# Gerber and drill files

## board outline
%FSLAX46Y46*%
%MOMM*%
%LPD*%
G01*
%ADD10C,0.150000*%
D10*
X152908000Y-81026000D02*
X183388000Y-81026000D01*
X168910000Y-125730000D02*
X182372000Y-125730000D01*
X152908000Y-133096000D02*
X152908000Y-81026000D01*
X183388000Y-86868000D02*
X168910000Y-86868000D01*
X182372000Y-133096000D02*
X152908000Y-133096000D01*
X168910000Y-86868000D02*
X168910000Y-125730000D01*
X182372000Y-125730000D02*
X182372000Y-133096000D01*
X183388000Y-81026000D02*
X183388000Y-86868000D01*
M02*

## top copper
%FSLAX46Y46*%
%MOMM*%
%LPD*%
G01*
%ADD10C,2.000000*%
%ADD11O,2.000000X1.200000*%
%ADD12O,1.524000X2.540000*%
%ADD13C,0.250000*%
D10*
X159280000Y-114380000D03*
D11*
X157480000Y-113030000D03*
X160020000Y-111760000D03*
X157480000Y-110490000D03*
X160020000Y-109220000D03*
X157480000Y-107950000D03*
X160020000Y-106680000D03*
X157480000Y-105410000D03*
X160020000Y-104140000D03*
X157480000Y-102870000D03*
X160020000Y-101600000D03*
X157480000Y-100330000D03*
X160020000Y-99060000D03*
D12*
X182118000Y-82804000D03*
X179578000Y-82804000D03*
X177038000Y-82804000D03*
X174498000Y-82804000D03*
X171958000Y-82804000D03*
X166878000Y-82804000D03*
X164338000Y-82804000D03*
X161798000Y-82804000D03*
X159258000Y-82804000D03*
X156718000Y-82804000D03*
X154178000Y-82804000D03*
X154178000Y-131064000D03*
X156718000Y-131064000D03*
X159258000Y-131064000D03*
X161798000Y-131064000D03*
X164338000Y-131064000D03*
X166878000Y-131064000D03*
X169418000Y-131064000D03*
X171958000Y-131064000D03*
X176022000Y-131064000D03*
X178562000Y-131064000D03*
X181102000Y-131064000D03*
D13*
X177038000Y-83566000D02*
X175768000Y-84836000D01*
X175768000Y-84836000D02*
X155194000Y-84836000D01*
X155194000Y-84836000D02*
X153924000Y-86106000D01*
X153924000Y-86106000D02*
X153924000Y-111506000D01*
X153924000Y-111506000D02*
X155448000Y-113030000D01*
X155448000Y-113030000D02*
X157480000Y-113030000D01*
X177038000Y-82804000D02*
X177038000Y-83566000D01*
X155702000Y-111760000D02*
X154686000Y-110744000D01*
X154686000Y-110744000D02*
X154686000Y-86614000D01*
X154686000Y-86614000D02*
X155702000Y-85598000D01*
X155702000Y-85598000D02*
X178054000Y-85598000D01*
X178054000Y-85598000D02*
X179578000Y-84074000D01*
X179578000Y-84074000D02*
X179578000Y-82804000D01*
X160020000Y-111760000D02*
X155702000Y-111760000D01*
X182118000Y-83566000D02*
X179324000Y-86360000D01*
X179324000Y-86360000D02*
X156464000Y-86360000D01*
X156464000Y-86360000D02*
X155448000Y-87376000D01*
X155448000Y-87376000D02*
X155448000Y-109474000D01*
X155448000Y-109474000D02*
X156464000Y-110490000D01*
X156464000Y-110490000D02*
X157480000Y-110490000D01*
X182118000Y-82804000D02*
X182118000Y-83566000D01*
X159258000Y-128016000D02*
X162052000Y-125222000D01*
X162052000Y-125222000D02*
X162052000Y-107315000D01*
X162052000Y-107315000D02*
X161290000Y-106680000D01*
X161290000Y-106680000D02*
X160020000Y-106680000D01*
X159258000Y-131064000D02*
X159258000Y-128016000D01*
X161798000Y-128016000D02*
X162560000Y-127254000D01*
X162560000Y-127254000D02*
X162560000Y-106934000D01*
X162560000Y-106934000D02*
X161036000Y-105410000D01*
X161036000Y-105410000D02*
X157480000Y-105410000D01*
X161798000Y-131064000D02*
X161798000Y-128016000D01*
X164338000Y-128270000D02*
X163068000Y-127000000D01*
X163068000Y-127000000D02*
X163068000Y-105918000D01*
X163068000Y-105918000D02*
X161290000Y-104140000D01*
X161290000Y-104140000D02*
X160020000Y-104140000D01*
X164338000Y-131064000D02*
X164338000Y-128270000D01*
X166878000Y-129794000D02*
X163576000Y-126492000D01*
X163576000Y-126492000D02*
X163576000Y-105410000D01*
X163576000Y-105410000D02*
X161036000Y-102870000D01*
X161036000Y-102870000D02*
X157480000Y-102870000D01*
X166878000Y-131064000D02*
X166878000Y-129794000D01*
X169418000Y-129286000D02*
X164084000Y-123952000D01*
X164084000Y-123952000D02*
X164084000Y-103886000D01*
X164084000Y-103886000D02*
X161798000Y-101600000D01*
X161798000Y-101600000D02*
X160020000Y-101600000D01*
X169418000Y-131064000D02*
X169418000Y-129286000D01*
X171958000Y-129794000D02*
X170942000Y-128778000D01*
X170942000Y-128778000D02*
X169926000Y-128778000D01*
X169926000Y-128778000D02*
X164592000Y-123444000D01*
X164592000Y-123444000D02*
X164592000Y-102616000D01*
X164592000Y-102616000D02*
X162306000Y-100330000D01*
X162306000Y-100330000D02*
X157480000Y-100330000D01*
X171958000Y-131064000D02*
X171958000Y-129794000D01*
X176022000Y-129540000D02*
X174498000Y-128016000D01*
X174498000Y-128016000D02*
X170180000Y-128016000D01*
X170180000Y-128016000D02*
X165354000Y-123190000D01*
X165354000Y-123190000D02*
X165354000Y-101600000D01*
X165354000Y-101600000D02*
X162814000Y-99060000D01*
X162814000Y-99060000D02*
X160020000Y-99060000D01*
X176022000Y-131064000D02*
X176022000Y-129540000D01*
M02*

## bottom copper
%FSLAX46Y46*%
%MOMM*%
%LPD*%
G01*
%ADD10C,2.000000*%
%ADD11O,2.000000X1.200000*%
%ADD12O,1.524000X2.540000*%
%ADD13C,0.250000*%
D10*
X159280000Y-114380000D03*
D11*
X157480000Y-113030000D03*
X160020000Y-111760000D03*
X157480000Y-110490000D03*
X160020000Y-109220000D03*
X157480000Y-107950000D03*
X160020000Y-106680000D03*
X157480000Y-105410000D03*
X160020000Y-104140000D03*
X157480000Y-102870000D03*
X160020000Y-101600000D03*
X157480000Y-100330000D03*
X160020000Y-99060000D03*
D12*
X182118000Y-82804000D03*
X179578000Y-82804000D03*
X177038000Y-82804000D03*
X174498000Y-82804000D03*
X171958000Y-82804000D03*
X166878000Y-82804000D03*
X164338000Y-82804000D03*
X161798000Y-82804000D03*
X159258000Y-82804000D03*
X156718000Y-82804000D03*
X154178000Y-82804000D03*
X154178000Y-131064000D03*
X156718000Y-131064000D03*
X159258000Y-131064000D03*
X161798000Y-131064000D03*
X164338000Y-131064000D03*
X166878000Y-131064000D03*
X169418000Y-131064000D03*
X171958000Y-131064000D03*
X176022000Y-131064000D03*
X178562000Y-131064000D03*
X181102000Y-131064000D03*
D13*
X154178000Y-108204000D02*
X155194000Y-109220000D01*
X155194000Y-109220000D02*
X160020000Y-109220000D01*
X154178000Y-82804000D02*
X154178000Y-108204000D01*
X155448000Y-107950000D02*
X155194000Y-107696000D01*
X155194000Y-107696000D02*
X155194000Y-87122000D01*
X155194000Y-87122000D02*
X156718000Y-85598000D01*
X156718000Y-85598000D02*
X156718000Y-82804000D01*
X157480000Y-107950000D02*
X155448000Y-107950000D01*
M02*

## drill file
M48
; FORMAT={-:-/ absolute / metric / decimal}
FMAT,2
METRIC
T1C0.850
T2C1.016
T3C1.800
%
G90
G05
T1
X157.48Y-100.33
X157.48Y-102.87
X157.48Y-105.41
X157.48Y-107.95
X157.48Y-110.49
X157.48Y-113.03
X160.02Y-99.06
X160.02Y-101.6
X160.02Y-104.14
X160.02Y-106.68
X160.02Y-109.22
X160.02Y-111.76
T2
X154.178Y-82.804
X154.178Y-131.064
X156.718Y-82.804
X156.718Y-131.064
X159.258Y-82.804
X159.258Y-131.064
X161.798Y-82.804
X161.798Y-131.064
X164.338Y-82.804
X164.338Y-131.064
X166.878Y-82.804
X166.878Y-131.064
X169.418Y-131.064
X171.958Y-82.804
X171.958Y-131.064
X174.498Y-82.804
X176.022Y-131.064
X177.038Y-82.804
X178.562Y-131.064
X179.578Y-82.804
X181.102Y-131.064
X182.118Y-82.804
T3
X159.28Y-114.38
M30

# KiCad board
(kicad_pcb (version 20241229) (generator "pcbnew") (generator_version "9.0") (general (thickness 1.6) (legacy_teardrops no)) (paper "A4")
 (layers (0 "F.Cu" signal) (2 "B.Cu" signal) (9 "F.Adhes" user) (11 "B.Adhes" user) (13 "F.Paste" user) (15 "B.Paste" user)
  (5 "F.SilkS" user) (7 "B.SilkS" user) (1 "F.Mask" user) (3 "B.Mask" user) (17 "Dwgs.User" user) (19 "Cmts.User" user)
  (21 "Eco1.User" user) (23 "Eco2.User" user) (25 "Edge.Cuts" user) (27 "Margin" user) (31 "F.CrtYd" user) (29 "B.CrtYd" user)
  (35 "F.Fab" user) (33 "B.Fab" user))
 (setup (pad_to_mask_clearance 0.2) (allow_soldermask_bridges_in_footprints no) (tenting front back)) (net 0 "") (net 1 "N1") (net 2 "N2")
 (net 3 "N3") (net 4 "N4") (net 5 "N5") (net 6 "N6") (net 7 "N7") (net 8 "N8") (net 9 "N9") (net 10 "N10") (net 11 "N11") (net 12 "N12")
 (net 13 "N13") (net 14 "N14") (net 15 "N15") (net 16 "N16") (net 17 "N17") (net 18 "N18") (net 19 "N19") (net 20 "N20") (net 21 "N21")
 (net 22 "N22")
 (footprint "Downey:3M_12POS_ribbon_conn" (layer "F.Cu") (at 158.75 106.68 90)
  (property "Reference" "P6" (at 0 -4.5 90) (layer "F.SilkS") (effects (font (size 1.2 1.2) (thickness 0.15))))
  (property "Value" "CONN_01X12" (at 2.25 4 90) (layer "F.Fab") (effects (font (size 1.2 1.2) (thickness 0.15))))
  (pad "" np_thru_hole circle (at -7.7 0.53 90) (size 2 2) (drill 1.8) (layers "*.Cu" "*.Mask"))
  (pad "1" thru_hole oval (at -6.35 -1.27 90) (size 1.2 2) (drill 0.85) (layers "*.Cu" "*.Mask") (remove_unused_layers no) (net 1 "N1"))
  (pad "2" thru_hole oval (at -5.08 1.27 90) (size 1.2 2) (drill 0.85) (layers "*.Cu" "*.Mask") (remove_unused_layers no) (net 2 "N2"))
  (pad "3" thru_hole oval (at -3.81 -1.27 90) (size 1.2 2) (drill 0.85) (layers "*.Cu" "*.Mask") (remove_unused_layers no) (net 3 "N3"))
  (pad "4" thru_hole oval (at -2.54 1.27 90) (size 1.2 2) (drill 0.85) (layers "*.Cu" "*.Mask") (remove_unused_layers no) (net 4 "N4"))
  (pad "5" thru_hole oval (at -1.27 -1.27 90) (size 1.2 2) (drill 0.85) (layers "*.Cu" "*.Mask") (remove_unused_layers no) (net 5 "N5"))
  (pad "6" thru_hole oval (at 0 1.27 90) (size 1.2 2) (drill 0.85) (layers "*.Cu" "*.Mask") (remove_unused_layers no) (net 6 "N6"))
  (pad "7" thru_hole oval (at 1.27 -1.27 90) (size 1.2 2) (drill 0.85) (layers "*.Cu" "*.Mask") (remove_unused_layers no) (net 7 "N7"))
  (pad "8" thru_hole oval (at 2.54 1.27 90) (size 1.2 2) (drill 0.85) (layers "*.Cu" "*.Mask") (remove_unused_layers no) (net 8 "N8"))
  (pad "9" thru_hole oval (at 3.81 -1.27 90) (size 1.2 2) (drill 0.85) (layers "*.Cu" "*.Mask") (remove_unused_layers no) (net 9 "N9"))
  (pad "10" thru_hole oval (at 5.08 1.27 90) (size 1.2 2) (drill 0.85) (layers "*.Cu" "*.Mask") (remove_unused_layers no) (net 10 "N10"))
  (pad "11" thru_hole oval (at 6.35 -1.27 90) (size 1.2 2) (drill 0.85) (layers "*.Cu" "*.Mask") (remove_unused_layers no) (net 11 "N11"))
  (pad "12" thru_hole oval (at 7.62 1.27 90) (size 1.2 2) (drill 0.85) (layers "*.Cu" "*.Mask") (remove_unused_layers no) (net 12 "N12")))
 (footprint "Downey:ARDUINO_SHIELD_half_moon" (layer "F.Cu") (at 148.59 104.14 -90)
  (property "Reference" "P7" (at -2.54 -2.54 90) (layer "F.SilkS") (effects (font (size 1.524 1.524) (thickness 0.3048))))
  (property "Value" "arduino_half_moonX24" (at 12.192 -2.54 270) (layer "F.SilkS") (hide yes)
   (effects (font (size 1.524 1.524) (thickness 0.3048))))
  (pad "1" thru_hole oval (at -21.336 -33.528 270) (size 2.54 1.524) (drill 1.016) (layers "*.Cu" "*.Mask" "F.SilkS")
   (remove_unused_layers no) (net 3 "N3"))
  (pad "2" thru_hole oval (at -21.336 -30.988 270) (size 2.54 1.524) (drill 1.016) (layers "*.Cu" "*.Mask" "F.SilkS")
   (remove_unused_layers no) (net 2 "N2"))
  (pad "3" thru_hole oval (at -21.336 -28.448 270) (size 2.54 1.524) (drill 1.016) (layers "*.Cu" "*.Mask" "F.SilkS")
   (remove_unused_layers no) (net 1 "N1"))
  (pad "4" thru_hole oval (at -21.336 -25.908 270) (size 2.54 1.524) (drill 1.016) (layers "*.Cu" "*.Mask" "F.SilkS")
   (remove_unused_layers no) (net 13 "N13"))
  (pad "5" thru_hole oval (at -21.336 -23.368 270) (size 2.54 1.524) (drill 1.016) (layers "*.Cu" "*.Mask" "F.SilkS")
   (remove_unused_layers no) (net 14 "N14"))
  (pad "6" thru_hole oval (at -21.336 -18.288 270) (size 2.54 1.524) (drill 1.016) (layers "*.Cu" "*.Mask" "F.SilkS")
   (remove_unused_layers no) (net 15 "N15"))
  (pad "7" thru_hole oval (at -21.336 -15.748 270) (size 2.54 1.524) (drill 1.016) (layers "*.Cu" "*.Mask" "F.SilkS")
   (remove_unused_layers no) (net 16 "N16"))
  (pad "8" thru_hole oval (at -21.336 -13.208 270) (size 2.54 1.524) (drill 1.016) (layers "*.Cu" "*.Mask" "F.SilkS")
   (remove_unused_layers no) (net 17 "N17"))
  (pad "9" thru_hole oval (at -21.336 -10.668 270) (size 2.54 1.524) (drill 1.016) (layers "*.Cu" "*.Mask" "F.SilkS")
   (remove_unused_layers no) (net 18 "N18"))
  (pad "10" thru_hole oval (at -21.336 -8.128 270) (size 2.54 1.524) (drill 1.016) (layers "*.Cu" "*.Mask" "F.SilkS")
   (remove_unused_layers no) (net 5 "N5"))
  (pad "11" thru_hole oval (at -21.336 -5.588 270) (size 2.54 1.524) (drill 1.016) (layers "*.Cu" "*.Mask" "F.SilkS")
   (remove_unused_layers no) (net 4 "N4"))
  (pad "12" thru_hole oval (at 26.924 -5.588 270) (size 2.54 1.524) (drill 1.016) (layers "*.Cu" "*.Mask" "F.SilkS")
   (remove_unused_layers no) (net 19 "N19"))
  (pad "13" thru_hole oval (at 26.924 -8.128 270) (size 2.54 1.524) (drill 1.016) (layers "*.Cu" "*.Mask" "F.SilkS")
   (remove_unused_layers no) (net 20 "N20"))
  (pad "14" thru_hole oval (at 26.924 -10.668 270) (size 2.54 1.524) (drill 1.016) (layers "*.Cu" "*.Mask" "F.SilkS")
   (remove_unused_layers no) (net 6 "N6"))
  (pad "15" thru_hole oval (at 26.924 -13.208 270) (size 2.54 1.524) (drill 1.016) (layers "*.Cu" "*.Mask" "F.SilkS")
   (remove_unused_layers no) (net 7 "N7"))
  (pad "16" thru_hole oval (at 26.924 -15.748 270) (size 2.54 1.524) (drill 1.016) (layers "*.Cu" "*.Mask" "F.SilkS")
   (remove_unused_layers no) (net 8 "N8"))
  (pad "17" thru_hole oval (at 26.924 -18.288 270) (size 2.54 1.524) (drill 1.016) (layers "*.Cu" "*.Mask" "F.SilkS")
   (remove_unused_layers no) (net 9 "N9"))
  (pad "18" thru_hole oval (at 26.924 -20.828 270) (size 2.54 1.524) (drill 1.016) (layers "*.Cu" "*.Mask" "F.SilkS")
   (remove_unused_layers no) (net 10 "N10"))
  (pad "19" thru_hole oval (at 26.924 -23.368 270) (size 2.54 1.524) (drill 1.016) (layers "*.Cu" "*.Mask" "F.SilkS")
   (remove_unused_layers no) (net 11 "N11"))
  (pad "20" thru_hole oval (at 26.924 -27.432 270) (size 2.54 1.524) (drill 1.016) (layers "*.Cu" "*.Mask" "F.SilkS")
   (remove_unused_layers no) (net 12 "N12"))
  (pad "21" thru_hole oval (at 26.924 -29.972 270) (size 2.54 1.524) (drill 1.016) (layers "*.Cu" "*.Mask" "F.SilkS")
   (remove_unused_layers no) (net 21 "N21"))
  (pad "22" thru_hole oval (at 26.924 -32.512 270) (size 2.54 1.524) (drill 1.016) (layers "*.Cu" "*.Mask" "F.SilkS")
   (remove_unused_layers no) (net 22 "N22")))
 (gr_line (start 152.908 81.026) (end 183.388 81.026) (stroke (width 0.15) (type solid)) (layer "Edge.Cuts"))
 (gr_line (start 168.91 125.73) (end 182.372 125.73) (stroke (width 0.15) (type solid)) (layer "Edge.Cuts"))
 (gr_line (start 152.908 133.096) (end 152.908 81.026) (stroke (width 0.15) (type solid)) (layer "Edge.Cuts"))
 (gr_line (start 183.388 86.868) (end 168.91 86.868) (stroke (width 0.15) (type solid)) (layer "Edge.Cuts"))
 (gr_line (start 182.372 133.096) (end 152.908 133.096) (stroke (width 0.15) (type solid)) (layer "Edge.Cuts"))
 (gr_line (start 168.91 86.868) (end 168.91 125.73) (stroke (width 0.15) (type solid)) (layer "Edge.Cuts"))
 (gr_line (start 182.372 125.73) (end 182.372 133.096) (stroke (width 0.15) (type solid)) (layer "Edge.Cuts"))
 (gr_line (start 183.388 81.026) (end 183.388 86.868) (stroke (width 0.15) (type solid)) (layer "Edge.Cuts"))
 (segment (start 177.038 83.566) (end 175.768 84.836) (width 0.25) (layer "F.Cu") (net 1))
 (segment (start 175.768 84.836) (end 155.194 84.836) (width 0.25) (layer "F.Cu") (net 1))
 (segment (start 155.194 84.836) (end 153.924 86.106) (width 0.25) (layer "F.Cu") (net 1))
 (segment (start 153.924 86.106) (end 153.924 111.506) (width 0.25) (layer "F.Cu") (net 1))
 (segment (start 153.924 111.506) (end 155.448 113.03) (width 0.25) (layer "F.Cu") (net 1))
 (segment (start 155.448 113.03) (end 157.48 113.03) (width 0.25) (layer "F.Cu") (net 1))
 (segment (start 177.038 82.804) (end 177.038 83.566) (width 0.25) (layer "F.Cu") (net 1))
 (segment (start 155.702 111.76) (end 154.686 110.744) (width 0.25) (layer "F.Cu") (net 2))
 (segment (start 154.686 110.744) (end 154.686 86.614) (width 0.25) (layer "F.Cu") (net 2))
 (segment (start 154.686 86.614) (end 155.702 85.598) (width 0.25) (layer "F.Cu") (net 2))
 (segment (start 155.702 85.598) (end 178.054 85.598) (width 0.25) (layer "F.Cu") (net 2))
 (segment (start 178.054 85.598) (end 179.578 84.074) (width 0.25) (layer "F.Cu") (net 2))
 (segment (start 179.578 84.074) (end 179.578 82.804) (width 0.25) (layer "F.Cu") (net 2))
 (segment (start 160.02 111.76) (end 155.702 111.76) (width 0.25) (layer "F.Cu") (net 2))
 (segment (start 182.118 83.566) (end 179.324 86.36) (width 0.25) (layer "F.Cu") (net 3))
 (segment (start 179.324 86.36) (end 156.464 86.36) (width 0.25) (layer "F.Cu") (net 3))
 (segment (start 156.464 86.36) (end 155.448 87.376) (width 0.25) (layer "F.Cu") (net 3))
 (segment (start 155.448 87.376) (end 155.448 109.474) (width 0.25) (layer "F.Cu") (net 3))
 (segment (start 155.448 109.474) (end 156.464 110.49) (width 0.25) (layer "F.Cu") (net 3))
 (segment (start 156.464 110.49) (end 157.48 110.49) (width 0.25) (layer "F.Cu") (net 3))
 (segment (start 182.118 82.804) (end 182.118 83.566) (width 0.25) (layer "F.Cu") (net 3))
 (segment (start 154.178 108.204) (end 155.194 109.22) (width 0.25) (layer "B.Cu") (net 4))
 (segment (start 155.194 109.22) (end 160.02 109.22) (width 0.25) (layer "B.Cu") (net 4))
 (segment (start 154.178 82.804) (end 154.178 108.204) (width 0.25) (layer "B.Cu") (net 4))
 (segment (start 155.448 107.95) (end 155.194 107.696) (width 0.25) (layer "B.Cu") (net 5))
 (segment (start 155.194 107.696) (end 155.194 87.122) (width 0.25) (layer "B.Cu") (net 5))
 (segment (start 155.194 87.122) (end 156.718 85.598) (width 0.25) (layer "B.Cu") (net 5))
 (segment (start 156.718 85.598) (end 156.718 82.804) (width 0.25) (layer "B.Cu") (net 5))
 (segment (start 157.48 107.95) (end 155.448 107.95) (width 0.25) (layer "B.Cu") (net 5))
 (segment (start 159.258 128.016) (end 162.052 125.222) (width 0.25) (layer "F.Cu") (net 6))
 (segment (start 162.052 125.222) (end 162.052 107.315) (width 0.25) (layer "F.Cu") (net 6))
 (segment (start 162.052 107.315) (end 161.29 106.68) (width 0.25) (layer "F.Cu") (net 6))
 (segment (start 161.29 106.68) (end 160.02 106.68) (width 0.25) (layer "F.Cu") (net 6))
 (segment (start 159.258 131.064) (end 159.258 128.016) (width 0.25) (layer "F.Cu") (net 6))
 (segment (start 161.798 128.016) (end 162.56 127.254) (width 0.25) (layer "F.Cu") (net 7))
 (segment (start 162.56 127.254) (end 162.56 106.934) (width 0.25) (layer "F.Cu") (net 7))
 (segment (start 162.56 106.934) (end 161.036 105.41) (width 0.25) (layer "F.Cu") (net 7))
 (segment (start 161.036 105.41) (end 157.48 105.41) (width 0.25) (layer "F.Cu") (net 7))
 (segment (start 161.798 131.064) (end 161.798 128.016) (width 0.25) (layer "F.Cu") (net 7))
 (segment (start 164.338 128.27) (end 163.068 127) (width 0.25) (layer "F.Cu") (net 8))
 (segment (start 163.068 127) (end 163.068 105.918) (width 0.25) (layer "F.Cu") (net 8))
 (segment (start 163.068 105.918) (end 161.29 104.14) (width 0.25) (layer "F.Cu") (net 8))
 (segment (start 161.29 104.14) (end 160.02 104.14) (width 0.25) (layer "F.Cu") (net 8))
 (segment (start 164.338 131.064) (end 164.338 128.27) (width 0.25) (layer "F.Cu") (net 8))
 (segment (start 166.878 129.794) (end 163.576 126.492) (width 0.25) (layer "F.Cu") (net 9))
 (segment (start 163.576 126.492) (end 163.576 105.41) (width 0.25) (layer "F.Cu") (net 9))
 (segment (start 163.576 105.41) (end 161.036 102.87) (width 0.25) (layer "F.Cu") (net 9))
 (segment (start 161.036 102.87) (end 157.48 102.87) (width 0.25) (layer "F.Cu") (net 9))
 (segment (start 166.878 131.064) (end 166.878 129.794) (width 0.25) (layer "F.Cu") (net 9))
 (segment (start 169.418 129.286) (end 164.084 123.952) (width 0.25) (layer "F.Cu") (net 10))
 (segment (start 164.084 123.952) (end 164.084 103.886) (width 0.25) (layer "F.Cu") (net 10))
 (segment (start 164.084 103.886) (end 161.798 101.6) (width 0.25) (layer "F.Cu") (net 10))
 (segment (start 161.798 101.6) (end 160.02 101.6) (width 0.25) (layer "F.Cu") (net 10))
 (segment (start 169.418 131.064) (end 169.418 129.286) (width 0.25) (layer "F.Cu") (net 10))
 (segment (start 171.958 129.794) (end 170.942 128.778) (width 0.25) (layer "F.Cu") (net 11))
 (segment (start 170.942 128.778) (end 169.926 128.778) (width 0.25) (layer "F.Cu") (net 11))
 (segment (start 169.926 128.778) (end 164.592 123.444) (width 0.25) (layer "F.Cu") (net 11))
 (segment (start 164.592 123.444) (end 164.592 102.616) (width 0.25) (layer "F.Cu") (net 11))
 (segment (start 164.592 102.616) (end 162.306 100.33) (width 0.25) (layer "F.Cu") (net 11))
 (segment (start 162.306 100.33) (end 157.48 100.33) (width 0.25) (layer "F.Cu") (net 11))
 (segment (start 171.958 131.064) (end 171.958 129.794) (width 0.25) (layer "F.Cu") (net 11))
 (segment (start 176.022 129.54) (end 174.498 128.016) (width 0.25) (layer "F.Cu") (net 12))
 (segment (start 174.498 128.016) (end 170.18 128.016) (width 0.25) (layer "F.Cu") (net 12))
 (segment (start 170.18 128.016) (end 165.354 123.19) (width 0.25) (layer "F.Cu") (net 12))
 (segment (start 165.354 123.19) (end 165.354 101.6) (width 0.25) (layer "F.Cu") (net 12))
 (segment (start 165.354 101.6) (end 162.814 99.06) (width 0.25) (layer "F.Cu") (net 12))
 (segment (start 162.814 99.06) (end 160.02 99.06) (width 0.25) (layer "F.Cu") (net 12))
 (segment (start 176.022 131.064) (end 176.022 129.54) (width 0.25) (layer "F.Cu") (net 12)))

